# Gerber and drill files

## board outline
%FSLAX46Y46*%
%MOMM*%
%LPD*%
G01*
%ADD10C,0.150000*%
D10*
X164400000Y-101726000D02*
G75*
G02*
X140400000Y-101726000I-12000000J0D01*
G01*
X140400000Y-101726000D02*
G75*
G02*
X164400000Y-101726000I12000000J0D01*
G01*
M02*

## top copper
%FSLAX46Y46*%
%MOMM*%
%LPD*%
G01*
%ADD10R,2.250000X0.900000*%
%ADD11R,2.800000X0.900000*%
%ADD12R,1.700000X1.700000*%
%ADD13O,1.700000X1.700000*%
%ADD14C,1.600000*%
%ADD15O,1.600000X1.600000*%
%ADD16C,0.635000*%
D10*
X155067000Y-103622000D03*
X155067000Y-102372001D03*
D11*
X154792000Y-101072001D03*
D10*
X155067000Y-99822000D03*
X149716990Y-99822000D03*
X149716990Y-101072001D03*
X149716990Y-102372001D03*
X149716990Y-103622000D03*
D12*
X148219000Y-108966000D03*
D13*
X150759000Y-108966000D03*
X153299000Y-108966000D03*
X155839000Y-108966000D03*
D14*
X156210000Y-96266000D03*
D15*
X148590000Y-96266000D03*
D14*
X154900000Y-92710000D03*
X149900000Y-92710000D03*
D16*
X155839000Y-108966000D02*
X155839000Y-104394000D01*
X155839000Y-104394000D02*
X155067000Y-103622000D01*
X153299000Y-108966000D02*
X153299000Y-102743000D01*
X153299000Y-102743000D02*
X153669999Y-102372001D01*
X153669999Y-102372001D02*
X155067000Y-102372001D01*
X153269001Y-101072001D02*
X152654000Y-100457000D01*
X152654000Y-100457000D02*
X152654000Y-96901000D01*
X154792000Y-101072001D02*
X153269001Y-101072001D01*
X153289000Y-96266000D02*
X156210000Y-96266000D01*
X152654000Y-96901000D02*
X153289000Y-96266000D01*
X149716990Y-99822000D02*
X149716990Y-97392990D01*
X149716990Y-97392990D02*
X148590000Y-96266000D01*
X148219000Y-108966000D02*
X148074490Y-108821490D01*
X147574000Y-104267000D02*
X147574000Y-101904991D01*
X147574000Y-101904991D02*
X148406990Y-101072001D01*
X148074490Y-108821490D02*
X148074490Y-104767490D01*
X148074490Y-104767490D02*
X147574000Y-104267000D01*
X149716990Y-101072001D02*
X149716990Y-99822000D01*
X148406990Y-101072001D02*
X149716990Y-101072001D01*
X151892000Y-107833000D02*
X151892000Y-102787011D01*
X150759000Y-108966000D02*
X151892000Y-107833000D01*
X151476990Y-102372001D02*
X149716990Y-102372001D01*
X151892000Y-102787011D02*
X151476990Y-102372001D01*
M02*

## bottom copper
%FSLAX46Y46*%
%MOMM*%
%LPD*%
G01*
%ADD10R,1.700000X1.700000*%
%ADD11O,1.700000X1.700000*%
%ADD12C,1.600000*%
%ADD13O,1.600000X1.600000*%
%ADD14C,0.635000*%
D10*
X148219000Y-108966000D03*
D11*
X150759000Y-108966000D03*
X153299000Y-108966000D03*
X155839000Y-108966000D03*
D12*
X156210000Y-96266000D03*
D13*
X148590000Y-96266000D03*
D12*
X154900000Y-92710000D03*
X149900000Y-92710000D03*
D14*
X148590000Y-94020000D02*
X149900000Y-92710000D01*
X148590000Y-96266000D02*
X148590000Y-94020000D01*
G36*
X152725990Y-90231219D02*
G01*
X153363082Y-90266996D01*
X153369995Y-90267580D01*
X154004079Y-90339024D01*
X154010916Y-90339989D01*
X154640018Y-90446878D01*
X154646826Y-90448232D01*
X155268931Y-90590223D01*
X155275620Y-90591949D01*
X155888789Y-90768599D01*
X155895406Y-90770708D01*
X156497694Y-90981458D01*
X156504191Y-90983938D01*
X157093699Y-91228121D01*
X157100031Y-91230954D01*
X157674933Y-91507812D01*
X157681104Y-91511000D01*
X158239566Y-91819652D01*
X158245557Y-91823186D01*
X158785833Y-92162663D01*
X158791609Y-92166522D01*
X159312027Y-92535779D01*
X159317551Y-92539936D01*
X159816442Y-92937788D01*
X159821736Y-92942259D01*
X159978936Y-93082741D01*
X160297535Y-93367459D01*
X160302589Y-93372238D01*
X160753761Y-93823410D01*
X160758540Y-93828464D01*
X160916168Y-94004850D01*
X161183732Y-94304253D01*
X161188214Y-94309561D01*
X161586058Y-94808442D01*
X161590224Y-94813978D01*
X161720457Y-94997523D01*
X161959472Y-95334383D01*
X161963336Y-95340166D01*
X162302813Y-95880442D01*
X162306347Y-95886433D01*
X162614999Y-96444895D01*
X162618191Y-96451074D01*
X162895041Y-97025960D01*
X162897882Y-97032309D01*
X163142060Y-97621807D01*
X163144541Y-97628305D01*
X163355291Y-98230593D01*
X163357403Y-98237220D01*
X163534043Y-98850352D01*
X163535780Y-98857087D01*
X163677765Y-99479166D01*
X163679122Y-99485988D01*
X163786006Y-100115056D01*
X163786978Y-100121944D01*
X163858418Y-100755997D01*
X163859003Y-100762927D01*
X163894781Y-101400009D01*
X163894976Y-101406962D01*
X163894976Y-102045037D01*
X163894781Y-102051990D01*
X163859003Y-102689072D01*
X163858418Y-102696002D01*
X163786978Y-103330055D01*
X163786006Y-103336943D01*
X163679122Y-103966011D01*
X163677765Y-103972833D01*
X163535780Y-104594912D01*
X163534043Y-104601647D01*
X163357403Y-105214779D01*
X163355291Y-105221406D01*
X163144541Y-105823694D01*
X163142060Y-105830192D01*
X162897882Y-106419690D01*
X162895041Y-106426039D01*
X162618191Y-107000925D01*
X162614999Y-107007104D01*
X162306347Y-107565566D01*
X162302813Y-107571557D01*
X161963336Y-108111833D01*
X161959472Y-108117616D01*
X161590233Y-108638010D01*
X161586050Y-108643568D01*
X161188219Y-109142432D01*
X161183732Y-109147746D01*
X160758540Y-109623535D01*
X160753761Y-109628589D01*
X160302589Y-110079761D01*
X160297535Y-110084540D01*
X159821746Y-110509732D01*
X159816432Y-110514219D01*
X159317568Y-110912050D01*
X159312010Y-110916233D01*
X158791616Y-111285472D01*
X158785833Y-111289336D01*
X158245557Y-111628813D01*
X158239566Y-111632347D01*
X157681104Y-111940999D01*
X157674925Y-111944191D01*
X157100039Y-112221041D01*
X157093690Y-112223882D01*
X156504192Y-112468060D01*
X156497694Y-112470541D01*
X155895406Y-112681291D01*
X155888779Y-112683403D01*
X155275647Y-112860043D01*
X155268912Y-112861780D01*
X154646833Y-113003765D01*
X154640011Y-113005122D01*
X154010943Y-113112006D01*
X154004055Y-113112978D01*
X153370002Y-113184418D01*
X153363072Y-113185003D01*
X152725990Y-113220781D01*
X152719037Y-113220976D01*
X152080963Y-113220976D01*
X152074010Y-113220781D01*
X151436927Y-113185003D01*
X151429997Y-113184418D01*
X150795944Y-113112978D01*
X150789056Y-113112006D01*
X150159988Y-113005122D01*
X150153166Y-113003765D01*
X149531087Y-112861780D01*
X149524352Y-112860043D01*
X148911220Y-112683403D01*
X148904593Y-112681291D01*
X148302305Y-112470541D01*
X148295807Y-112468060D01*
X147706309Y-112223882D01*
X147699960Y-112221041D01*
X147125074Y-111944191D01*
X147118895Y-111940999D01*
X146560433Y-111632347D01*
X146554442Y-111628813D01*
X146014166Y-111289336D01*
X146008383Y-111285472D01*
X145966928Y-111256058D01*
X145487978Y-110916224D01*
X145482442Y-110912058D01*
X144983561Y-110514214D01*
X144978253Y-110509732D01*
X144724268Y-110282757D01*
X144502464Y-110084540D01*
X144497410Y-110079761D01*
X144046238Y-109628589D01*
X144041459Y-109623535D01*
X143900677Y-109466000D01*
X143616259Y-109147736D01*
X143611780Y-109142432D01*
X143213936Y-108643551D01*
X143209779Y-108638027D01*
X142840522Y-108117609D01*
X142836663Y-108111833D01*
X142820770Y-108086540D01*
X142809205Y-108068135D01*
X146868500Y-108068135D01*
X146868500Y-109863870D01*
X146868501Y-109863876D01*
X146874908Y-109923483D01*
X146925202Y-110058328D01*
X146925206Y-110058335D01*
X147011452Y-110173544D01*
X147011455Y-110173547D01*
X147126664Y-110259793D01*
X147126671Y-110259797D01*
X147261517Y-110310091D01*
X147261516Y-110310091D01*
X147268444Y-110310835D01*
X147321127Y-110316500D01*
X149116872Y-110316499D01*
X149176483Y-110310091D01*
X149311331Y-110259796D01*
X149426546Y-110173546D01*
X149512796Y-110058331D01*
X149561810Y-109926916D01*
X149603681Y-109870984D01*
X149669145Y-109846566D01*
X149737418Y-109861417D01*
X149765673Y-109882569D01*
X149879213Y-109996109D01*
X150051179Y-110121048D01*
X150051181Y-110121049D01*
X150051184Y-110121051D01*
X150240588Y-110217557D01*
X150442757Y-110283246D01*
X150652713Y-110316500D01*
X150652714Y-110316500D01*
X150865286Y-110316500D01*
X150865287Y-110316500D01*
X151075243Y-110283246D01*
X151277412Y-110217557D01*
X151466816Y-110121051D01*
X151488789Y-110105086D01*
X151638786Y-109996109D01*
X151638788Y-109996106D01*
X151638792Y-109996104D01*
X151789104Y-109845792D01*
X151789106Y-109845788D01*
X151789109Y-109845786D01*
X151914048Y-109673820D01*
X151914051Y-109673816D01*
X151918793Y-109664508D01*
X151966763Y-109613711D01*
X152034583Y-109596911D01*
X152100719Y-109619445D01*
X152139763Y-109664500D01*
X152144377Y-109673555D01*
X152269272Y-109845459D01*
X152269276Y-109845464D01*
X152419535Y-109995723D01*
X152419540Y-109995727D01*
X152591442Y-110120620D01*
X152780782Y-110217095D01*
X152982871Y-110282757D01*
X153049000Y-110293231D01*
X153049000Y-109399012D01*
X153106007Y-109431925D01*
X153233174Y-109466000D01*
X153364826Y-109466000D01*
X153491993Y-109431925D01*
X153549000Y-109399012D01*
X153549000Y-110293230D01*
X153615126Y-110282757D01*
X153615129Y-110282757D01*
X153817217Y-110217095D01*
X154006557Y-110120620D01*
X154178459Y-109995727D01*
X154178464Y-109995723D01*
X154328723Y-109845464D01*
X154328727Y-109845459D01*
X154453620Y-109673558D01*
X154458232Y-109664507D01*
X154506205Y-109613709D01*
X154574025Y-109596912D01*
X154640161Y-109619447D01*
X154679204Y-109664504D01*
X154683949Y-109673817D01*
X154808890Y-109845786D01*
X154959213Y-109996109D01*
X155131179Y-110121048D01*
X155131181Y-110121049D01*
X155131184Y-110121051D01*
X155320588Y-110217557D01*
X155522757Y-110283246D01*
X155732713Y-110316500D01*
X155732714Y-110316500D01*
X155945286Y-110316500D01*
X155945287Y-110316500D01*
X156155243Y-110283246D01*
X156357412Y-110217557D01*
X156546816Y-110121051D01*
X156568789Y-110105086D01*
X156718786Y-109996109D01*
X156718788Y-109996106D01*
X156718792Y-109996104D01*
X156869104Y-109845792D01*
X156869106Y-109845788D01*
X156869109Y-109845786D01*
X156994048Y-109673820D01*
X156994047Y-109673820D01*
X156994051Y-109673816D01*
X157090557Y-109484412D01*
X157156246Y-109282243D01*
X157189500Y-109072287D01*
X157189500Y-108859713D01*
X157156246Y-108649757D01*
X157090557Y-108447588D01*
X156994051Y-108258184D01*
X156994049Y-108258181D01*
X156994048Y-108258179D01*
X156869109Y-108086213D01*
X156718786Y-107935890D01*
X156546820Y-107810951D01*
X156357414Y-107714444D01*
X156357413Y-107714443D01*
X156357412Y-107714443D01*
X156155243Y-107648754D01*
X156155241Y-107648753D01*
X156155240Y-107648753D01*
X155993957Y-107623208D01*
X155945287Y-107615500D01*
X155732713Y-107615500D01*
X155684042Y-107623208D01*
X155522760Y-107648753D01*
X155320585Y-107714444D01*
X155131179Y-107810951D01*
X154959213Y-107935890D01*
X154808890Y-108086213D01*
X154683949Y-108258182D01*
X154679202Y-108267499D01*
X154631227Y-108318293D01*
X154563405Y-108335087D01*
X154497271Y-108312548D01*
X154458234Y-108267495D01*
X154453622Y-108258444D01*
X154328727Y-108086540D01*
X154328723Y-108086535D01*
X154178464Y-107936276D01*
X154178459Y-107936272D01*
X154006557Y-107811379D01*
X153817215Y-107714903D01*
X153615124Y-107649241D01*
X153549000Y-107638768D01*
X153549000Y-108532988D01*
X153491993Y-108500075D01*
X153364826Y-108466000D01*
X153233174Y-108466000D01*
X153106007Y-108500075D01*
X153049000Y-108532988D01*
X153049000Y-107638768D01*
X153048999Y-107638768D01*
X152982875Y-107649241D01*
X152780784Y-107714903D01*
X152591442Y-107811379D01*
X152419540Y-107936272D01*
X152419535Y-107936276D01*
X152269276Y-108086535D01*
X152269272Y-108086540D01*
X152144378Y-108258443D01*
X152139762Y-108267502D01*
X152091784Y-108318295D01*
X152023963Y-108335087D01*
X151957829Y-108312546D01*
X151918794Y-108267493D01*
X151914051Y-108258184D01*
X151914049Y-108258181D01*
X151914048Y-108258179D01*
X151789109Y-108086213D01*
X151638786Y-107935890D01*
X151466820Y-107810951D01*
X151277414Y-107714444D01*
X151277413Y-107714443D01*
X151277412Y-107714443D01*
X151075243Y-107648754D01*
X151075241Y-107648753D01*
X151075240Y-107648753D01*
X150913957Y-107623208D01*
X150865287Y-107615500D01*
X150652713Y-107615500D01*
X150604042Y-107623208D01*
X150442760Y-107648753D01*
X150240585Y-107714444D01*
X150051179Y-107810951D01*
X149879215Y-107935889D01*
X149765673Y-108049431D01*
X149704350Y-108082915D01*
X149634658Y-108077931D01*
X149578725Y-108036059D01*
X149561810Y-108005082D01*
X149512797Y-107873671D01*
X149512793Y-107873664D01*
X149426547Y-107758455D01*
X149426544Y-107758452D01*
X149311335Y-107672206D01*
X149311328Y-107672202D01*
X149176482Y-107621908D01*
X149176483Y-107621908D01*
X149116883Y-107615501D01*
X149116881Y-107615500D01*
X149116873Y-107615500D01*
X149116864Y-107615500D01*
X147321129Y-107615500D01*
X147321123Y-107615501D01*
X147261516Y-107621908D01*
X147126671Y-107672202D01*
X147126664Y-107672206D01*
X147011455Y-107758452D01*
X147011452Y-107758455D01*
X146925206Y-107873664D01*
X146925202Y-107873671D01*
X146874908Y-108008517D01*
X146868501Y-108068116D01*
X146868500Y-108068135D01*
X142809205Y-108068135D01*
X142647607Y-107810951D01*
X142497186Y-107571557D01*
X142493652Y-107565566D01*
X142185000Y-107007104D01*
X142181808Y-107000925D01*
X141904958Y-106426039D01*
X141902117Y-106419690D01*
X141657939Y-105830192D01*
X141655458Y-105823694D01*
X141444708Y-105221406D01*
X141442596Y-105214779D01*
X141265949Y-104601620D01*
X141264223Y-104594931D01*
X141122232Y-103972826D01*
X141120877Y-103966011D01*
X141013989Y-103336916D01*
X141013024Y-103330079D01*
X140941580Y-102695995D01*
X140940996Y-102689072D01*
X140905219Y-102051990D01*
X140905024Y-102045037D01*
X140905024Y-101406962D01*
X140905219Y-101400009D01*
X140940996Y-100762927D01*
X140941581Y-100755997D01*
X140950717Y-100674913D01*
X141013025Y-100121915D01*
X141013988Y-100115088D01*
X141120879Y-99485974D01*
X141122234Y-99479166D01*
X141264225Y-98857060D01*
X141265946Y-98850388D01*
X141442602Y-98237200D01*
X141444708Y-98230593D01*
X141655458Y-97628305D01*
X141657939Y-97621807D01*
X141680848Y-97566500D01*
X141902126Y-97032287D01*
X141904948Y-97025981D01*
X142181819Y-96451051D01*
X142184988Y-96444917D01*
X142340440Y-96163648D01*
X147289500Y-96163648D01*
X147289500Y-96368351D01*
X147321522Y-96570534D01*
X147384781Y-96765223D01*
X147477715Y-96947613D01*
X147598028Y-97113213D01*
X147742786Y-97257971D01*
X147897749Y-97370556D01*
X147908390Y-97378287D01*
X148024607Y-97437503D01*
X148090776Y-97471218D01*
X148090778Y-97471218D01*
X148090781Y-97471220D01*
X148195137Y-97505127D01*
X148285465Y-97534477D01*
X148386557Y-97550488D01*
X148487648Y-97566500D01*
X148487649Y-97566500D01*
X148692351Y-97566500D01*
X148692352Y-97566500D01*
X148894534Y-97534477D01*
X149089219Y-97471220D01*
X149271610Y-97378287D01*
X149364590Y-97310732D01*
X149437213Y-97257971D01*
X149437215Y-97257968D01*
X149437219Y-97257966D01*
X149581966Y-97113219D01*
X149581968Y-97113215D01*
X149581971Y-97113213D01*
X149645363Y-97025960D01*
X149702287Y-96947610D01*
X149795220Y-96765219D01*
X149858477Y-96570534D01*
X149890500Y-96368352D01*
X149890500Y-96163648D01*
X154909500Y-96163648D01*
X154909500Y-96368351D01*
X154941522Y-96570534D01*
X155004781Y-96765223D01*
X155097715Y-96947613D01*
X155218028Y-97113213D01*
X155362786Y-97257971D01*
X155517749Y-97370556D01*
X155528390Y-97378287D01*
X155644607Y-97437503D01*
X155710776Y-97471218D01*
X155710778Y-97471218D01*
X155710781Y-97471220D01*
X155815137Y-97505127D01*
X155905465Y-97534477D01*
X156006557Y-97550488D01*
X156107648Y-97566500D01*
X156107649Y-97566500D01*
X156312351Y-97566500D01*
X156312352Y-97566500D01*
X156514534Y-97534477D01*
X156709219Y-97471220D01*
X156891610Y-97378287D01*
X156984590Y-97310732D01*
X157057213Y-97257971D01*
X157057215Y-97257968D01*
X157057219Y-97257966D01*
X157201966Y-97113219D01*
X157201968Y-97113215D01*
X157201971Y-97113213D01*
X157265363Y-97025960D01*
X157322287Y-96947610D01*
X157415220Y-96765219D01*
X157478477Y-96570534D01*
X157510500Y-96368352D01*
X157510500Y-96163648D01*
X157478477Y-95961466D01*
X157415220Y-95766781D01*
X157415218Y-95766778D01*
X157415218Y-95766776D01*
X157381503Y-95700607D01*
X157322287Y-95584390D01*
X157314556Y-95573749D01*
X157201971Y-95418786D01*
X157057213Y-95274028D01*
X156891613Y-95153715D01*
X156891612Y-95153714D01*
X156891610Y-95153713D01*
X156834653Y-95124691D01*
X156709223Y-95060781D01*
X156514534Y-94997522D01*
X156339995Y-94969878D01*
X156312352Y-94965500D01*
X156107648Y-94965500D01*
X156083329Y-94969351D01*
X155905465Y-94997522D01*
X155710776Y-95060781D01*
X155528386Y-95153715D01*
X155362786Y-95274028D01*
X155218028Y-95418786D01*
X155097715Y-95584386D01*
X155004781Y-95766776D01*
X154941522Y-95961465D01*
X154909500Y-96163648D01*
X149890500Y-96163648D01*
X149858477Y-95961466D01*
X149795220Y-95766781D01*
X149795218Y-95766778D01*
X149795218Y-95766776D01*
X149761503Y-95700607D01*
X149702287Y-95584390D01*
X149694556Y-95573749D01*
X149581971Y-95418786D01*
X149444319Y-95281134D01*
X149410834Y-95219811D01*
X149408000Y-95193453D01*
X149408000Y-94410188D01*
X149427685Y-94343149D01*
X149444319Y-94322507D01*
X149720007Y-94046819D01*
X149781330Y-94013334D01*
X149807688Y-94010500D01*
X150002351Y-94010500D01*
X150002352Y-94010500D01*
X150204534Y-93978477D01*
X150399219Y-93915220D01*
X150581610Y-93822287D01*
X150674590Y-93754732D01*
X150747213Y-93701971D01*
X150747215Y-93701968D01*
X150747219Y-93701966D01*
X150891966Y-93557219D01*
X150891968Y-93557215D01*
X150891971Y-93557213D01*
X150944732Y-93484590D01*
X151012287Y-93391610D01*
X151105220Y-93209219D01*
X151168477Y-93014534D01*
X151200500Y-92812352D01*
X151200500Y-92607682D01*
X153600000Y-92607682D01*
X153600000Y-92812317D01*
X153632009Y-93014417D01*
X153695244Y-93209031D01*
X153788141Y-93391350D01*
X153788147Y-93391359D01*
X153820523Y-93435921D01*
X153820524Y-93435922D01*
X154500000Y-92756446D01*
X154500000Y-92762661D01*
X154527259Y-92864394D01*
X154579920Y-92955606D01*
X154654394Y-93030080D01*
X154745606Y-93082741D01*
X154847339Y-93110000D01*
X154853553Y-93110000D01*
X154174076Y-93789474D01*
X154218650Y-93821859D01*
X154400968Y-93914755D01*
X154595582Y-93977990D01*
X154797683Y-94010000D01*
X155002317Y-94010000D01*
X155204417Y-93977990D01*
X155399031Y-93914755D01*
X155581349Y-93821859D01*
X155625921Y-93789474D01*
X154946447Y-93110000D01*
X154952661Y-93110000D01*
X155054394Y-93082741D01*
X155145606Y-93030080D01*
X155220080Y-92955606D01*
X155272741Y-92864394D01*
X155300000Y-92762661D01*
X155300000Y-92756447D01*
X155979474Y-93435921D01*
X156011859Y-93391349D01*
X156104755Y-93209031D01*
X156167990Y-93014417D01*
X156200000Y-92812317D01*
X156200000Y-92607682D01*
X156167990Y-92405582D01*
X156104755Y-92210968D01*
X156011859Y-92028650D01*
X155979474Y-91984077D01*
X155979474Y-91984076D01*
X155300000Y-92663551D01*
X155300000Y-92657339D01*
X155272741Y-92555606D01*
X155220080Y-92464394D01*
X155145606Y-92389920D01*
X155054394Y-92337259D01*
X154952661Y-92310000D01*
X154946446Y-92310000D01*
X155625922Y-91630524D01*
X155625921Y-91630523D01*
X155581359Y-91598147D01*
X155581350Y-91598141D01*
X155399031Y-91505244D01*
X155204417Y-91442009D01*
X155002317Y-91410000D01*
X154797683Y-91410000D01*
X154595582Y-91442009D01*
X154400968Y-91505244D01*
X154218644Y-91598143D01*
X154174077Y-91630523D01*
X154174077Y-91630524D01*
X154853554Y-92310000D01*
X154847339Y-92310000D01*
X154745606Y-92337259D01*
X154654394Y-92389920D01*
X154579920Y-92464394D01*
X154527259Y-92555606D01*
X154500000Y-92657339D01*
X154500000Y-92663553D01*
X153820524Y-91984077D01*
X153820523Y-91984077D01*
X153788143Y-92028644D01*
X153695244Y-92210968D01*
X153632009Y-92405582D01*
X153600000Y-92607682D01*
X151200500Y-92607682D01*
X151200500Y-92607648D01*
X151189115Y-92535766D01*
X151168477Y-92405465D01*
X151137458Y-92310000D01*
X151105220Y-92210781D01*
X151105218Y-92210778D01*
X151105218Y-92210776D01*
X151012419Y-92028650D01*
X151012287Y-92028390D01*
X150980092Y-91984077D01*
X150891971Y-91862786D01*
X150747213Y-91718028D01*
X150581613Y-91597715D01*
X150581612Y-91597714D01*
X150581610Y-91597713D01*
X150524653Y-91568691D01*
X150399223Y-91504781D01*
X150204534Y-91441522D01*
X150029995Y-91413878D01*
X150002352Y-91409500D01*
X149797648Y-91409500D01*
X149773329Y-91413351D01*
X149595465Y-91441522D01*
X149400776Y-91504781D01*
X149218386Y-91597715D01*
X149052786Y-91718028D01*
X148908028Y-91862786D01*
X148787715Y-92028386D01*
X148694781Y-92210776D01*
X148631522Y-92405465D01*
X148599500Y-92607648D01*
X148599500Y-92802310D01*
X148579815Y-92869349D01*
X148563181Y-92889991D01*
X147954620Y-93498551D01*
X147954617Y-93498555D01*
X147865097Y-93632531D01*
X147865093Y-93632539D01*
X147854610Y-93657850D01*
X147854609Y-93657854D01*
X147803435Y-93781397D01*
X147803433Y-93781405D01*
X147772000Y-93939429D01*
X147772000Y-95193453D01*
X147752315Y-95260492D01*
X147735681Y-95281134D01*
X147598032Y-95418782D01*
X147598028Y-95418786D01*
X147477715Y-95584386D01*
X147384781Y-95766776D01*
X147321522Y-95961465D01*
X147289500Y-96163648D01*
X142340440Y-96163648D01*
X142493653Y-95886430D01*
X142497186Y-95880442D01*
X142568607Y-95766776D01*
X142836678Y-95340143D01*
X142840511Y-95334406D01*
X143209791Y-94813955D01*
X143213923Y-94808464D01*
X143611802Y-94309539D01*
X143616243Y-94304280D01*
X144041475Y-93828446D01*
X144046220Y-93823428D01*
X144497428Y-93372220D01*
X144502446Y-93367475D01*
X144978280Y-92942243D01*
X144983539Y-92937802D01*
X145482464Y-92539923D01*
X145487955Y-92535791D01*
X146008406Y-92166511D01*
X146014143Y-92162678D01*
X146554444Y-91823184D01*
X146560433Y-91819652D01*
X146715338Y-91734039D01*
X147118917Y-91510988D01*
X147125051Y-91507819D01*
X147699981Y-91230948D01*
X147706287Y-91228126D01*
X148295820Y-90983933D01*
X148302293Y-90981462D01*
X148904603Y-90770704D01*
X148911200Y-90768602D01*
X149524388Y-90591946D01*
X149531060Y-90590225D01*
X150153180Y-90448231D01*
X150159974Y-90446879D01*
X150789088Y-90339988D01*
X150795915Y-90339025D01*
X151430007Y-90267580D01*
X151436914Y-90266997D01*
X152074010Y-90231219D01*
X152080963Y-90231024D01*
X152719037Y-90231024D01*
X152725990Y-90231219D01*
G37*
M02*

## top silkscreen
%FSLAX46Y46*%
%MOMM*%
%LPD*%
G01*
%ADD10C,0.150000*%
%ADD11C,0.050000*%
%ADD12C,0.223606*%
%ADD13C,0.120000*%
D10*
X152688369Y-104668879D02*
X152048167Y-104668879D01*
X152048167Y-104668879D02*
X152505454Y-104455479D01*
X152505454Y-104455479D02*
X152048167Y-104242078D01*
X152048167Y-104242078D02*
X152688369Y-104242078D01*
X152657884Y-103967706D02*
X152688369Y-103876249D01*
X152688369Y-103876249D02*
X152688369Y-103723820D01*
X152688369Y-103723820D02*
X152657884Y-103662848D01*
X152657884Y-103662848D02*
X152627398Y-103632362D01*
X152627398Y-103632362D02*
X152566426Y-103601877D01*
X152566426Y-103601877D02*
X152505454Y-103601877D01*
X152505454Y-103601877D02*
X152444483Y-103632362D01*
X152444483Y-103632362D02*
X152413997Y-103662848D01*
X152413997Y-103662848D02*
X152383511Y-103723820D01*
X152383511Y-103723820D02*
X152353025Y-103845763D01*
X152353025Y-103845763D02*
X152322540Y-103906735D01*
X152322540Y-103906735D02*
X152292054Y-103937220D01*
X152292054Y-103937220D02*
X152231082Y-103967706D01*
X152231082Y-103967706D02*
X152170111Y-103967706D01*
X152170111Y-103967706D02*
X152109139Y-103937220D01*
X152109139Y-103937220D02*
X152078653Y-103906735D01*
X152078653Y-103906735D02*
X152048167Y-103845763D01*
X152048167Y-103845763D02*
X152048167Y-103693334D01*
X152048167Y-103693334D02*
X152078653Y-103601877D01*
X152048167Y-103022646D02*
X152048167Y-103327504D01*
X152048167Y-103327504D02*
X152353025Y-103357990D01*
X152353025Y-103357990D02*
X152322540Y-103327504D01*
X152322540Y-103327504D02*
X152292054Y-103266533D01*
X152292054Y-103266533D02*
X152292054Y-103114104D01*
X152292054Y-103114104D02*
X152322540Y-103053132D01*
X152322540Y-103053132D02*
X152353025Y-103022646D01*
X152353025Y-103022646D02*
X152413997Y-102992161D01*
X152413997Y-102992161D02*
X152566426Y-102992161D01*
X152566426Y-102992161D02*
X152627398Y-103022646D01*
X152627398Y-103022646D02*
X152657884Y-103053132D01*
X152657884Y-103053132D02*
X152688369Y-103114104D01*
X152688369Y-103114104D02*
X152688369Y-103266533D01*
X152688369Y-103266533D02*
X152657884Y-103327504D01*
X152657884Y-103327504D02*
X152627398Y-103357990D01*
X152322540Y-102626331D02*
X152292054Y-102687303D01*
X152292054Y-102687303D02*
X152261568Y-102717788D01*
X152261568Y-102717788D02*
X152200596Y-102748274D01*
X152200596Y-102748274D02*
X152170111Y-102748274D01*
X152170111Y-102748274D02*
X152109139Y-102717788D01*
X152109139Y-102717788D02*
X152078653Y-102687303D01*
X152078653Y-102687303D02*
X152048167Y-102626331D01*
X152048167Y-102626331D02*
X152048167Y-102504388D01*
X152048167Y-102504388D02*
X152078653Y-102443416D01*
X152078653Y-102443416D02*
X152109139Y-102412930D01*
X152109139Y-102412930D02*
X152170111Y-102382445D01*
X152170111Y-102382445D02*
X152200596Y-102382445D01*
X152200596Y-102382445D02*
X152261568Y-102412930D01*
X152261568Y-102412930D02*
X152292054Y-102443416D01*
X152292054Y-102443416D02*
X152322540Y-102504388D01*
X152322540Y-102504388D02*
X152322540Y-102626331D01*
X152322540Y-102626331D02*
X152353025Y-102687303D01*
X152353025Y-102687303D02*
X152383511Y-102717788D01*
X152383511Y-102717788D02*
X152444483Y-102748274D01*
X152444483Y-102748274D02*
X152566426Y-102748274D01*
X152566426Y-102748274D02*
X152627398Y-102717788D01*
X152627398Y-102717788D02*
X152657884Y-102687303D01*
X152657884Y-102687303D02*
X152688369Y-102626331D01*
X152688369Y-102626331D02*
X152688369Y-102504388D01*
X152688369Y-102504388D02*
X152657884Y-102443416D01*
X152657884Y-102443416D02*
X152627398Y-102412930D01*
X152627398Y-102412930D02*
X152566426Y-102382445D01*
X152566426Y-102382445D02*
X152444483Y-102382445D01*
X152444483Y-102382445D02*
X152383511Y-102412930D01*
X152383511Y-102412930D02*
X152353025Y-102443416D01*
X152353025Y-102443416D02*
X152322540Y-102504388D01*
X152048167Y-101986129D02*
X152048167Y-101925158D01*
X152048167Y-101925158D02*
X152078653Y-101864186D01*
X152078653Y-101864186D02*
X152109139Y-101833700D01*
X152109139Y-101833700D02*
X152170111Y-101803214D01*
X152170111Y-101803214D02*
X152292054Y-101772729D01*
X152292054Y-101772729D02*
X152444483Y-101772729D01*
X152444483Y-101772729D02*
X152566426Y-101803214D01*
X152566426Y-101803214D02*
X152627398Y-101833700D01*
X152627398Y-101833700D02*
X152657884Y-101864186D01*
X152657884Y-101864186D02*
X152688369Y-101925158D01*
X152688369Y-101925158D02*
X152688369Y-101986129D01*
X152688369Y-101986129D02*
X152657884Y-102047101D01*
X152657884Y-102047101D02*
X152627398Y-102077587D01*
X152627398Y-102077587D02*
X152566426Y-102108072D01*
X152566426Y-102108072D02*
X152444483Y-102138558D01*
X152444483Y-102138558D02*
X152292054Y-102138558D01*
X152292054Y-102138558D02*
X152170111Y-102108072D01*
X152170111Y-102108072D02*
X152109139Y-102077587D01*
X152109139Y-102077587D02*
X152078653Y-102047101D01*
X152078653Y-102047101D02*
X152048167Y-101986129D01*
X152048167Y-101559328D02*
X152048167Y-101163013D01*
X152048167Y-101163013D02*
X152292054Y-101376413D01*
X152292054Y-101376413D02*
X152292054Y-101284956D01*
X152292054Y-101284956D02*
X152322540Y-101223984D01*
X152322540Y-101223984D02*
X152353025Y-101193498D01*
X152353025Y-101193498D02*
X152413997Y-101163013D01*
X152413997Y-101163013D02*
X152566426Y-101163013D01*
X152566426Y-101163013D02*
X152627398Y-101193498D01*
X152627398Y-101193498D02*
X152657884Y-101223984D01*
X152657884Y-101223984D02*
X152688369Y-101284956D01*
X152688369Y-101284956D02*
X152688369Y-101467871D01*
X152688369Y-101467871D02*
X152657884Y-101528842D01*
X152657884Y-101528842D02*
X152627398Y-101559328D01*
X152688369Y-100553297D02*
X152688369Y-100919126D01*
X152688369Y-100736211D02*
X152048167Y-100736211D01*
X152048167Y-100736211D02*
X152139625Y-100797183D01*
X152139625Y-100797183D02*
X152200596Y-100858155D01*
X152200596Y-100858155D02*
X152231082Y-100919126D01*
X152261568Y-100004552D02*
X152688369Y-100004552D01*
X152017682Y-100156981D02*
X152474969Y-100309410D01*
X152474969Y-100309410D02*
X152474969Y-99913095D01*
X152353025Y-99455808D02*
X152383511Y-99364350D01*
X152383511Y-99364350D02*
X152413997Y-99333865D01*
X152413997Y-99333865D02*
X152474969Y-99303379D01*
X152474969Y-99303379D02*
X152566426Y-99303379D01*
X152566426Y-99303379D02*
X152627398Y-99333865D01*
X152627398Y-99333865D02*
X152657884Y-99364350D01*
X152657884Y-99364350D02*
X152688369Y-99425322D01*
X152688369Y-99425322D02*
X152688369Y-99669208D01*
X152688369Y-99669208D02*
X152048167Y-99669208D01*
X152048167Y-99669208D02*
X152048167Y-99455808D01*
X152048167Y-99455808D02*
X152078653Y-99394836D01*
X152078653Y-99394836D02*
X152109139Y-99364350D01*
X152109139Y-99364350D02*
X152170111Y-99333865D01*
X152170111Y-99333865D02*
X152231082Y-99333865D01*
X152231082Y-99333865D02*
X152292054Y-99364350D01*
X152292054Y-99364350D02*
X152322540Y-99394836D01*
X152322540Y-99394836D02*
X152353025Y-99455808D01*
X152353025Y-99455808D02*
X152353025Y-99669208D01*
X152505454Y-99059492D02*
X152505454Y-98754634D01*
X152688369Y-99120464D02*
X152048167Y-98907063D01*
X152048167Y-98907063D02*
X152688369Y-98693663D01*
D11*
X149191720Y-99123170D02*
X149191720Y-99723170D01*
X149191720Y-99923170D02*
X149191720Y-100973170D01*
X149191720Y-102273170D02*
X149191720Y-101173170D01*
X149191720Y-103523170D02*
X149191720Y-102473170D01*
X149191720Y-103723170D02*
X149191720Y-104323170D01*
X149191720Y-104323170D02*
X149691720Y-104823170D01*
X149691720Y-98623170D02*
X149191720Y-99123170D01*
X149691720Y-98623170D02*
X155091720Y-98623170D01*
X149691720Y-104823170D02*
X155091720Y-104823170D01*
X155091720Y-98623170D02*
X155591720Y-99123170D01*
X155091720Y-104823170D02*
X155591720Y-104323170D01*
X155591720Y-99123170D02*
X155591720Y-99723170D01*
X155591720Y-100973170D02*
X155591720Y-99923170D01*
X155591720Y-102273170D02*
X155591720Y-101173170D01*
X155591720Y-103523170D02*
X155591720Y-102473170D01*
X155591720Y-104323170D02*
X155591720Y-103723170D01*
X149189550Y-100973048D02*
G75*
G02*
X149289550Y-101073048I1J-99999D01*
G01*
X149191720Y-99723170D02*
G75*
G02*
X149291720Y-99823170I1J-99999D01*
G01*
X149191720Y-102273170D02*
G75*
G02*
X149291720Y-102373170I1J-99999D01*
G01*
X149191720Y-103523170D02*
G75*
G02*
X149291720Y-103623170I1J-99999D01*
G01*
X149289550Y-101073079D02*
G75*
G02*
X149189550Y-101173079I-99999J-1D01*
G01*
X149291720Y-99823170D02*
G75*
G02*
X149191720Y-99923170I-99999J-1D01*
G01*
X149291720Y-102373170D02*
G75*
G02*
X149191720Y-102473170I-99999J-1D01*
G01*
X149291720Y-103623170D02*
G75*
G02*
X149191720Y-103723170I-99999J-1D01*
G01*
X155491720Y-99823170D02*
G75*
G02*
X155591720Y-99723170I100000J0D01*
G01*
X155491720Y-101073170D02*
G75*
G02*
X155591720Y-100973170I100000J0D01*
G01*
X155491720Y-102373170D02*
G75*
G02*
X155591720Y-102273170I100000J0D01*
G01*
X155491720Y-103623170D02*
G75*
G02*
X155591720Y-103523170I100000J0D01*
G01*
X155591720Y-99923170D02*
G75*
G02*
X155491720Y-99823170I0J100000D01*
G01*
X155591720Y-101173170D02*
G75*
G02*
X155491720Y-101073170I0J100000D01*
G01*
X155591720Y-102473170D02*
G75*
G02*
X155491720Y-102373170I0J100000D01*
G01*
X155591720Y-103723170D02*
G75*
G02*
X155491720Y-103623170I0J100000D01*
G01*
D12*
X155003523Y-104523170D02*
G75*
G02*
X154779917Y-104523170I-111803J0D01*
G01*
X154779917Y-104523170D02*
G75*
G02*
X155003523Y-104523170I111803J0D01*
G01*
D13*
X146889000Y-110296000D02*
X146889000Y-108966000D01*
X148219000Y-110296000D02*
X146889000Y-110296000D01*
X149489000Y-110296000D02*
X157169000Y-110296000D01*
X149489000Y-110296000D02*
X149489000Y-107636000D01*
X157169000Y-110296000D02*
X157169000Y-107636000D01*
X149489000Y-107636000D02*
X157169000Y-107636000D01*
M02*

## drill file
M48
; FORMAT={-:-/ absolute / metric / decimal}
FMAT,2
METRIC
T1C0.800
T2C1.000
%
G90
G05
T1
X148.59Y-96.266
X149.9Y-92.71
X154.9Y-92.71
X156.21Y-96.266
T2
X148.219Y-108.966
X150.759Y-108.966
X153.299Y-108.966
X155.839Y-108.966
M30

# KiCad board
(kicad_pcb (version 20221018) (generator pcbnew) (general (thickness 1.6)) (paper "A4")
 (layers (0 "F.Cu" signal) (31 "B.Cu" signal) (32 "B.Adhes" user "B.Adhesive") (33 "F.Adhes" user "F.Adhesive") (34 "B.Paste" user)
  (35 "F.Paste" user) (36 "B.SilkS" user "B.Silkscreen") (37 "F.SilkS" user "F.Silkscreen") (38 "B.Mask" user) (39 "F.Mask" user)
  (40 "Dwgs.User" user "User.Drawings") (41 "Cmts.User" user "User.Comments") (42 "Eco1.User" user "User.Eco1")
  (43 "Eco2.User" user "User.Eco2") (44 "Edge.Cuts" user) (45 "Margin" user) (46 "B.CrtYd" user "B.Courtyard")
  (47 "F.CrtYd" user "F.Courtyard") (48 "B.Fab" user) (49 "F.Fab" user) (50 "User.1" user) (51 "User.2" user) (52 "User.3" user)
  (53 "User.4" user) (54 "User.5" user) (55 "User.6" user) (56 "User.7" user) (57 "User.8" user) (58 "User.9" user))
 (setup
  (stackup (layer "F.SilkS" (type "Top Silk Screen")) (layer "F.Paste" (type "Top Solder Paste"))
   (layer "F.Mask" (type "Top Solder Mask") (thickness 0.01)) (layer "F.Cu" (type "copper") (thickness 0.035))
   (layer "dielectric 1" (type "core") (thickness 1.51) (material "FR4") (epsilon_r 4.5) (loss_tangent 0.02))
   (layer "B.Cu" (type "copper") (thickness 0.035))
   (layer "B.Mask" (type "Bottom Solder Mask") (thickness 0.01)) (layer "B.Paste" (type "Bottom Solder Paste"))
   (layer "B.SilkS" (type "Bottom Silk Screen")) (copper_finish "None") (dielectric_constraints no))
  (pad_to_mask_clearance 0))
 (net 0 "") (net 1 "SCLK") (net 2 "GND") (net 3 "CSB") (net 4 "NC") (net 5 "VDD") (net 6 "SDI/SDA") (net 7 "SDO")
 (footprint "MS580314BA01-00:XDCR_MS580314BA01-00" (layer "F.Cu") (at 152.39172 101.72317)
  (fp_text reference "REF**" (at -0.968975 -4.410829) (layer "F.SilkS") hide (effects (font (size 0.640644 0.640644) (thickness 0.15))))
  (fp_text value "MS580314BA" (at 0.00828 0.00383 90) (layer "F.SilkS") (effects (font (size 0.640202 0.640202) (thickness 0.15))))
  (fp_line (start -3.2 -2.6) (end -3.2 -2) (stroke (width 0.05) (type solid)) (layer "F.SilkS"))
  (fp_line (start -3.2 -1.8) (end -3.2 -0.75) (stroke (width 0.05) (type solid)) (layer "F.SilkS"))
  (fp_line (start -3.2 0.55) (end -3.2 -0.55) (stroke (width 0.05) (type solid)) (layer "F.SilkS"))
  (fp_line (start -3.2 1.8) (end -3.2 0.75) (stroke (width 0.05) (type solid)) (layer "F.SilkS"))
  (fp_line (start -3.2 2) (end -3.2 2.6) (stroke (width 0.05) (type solid)) (layer "F.SilkS"))
  (fp_line (start -3.2 2.6) (end -2.7 3.1) (stroke (width 0.05) (type solid)) (layer "F.SilkS"))
  (fp_line (start -2.7 -3.1) (end -3.2 -2.6) (stroke (width 0.05) (type solid)) (layer "F.SilkS"))
  (fp_line (start -2.7 -3.1) (end 2.7 -3.1) (stroke (width 0.05) (type solid)) (layer "F.SilkS"))
  (fp_line (start -2.7 3.1) (end 2.7 3.1) (stroke (width 0.05) (type solid)) (layer "F.SilkS"))
  (fp_line (start 2.7 -3.1) (end 3.2 -2.6) (stroke (width 0.05) (type solid)) (layer "F.SilkS"))
  (fp_line (start 2.7 3.1) (end 3.2 2.6) (stroke (width 0.05) (type solid)) (layer "F.SilkS"))
  (fp_line (start 3.2 -2.6) (end 3.2 -2) (stroke (width 0.05) (type solid)) (layer "F.SilkS"))
  (fp_line (start 3.2 -0.75) (end 3.2 -1.8) (stroke (width 0.05) (type solid)) (layer "F.SilkS"))
  (fp_line (start 3.2 0.55) (end 3.2 -0.55) (stroke (width 0.05) (type solid)) (layer "F.SilkS"))
  (fp_line (start 3.2 1.8) (end 3.2 0.75) (stroke (width 0.05) (type solid)) (layer "F.SilkS"))
  (fp_line (start 3.2 2.6) (end 3.2 2) (stroke (width 0.05) (type solid)) (layer "F.SilkS"))
  (fp_arc (start -3.20217 -0.750122) (mid -3.131459 -0.720833) (end -3.10217 -0.650122) (stroke (width 0.05) (type solid)) (layer "F.SilkS"))
  (fp_arc (start -3.2 -2) (mid -3.129289 -1.970711) (end -3.1 -1.9) (stroke (width 0.05) (type solid)) (layer "F.SilkS"))
  (fp_arc (start -3.2 0.55) (mid -3.129289 0.579289) (end -3.1 0.65) (stroke (width 0.05) (type solid)) (layer "F.SilkS"))
  (fp_arc (start -3.2 1.8) (mid -3.129289 1.829289) (end -3.1 1.9) (stroke (width 0.05) (type solid)) (layer "F.SilkS"))
  (fp_arc (start -3.10217 -0.650091) (mid -3.131459 -0.57938) (end -3.20217 -0.550091) (stroke (width 0.05) (type solid)) (layer "F.SilkS"))
  (fp_arc (start -3.1 -1.9) (mid -3.129289 -1.829289) (end -3.2 -1.8) (stroke (width 0.05) (type solid)) (layer "F.SilkS"))
  (fp_arc (start -3.1 0.65) (mid -3.129289 0.720711) (end -3.2 0.75) (stroke (width 0.05) (type solid)) (layer "F.SilkS"))
  (fp_arc (start -3.1 1.9) (mid -3.129289 1.970711) (end -3.2 2) (stroke (width 0.05) (type solid)) (layer "F.SilkS"))
  (fp_arc (start 3.1 -1.9) (mid 3.129289 -1.970711) (end 3.2 -2) (stroke (width 0.05) (type solid)) (layer "F.SilkS"))
  (fp_arc (start 3.1 -0.65) (mid 3.129289 -0.720711) (end 3.2 -0.75) (stroke (width 0.05) (type solid)) (layer "F.SilkS"))
  (fp_arc (start 3.1 0.65) (mid 3.129289 0.579289) (end 3.2 0.55) (stroke (width 0.05) (type solid)) (layer "F.SilkS"))
  (fp_arc (start 3.1 1.9) (mid 3.129289 1.829289) (end 3.2 1.8) (stroke (width 0.05) (type solid)) (layer "F.SilkS"))
  (fp_arc (start 3.2 -1.8) (mid 3.129289 -1.829289) (end 3.1 -1.9) (stroke (width 0.05) (type solid)) (layer "F.SilkS"))
  (fp_arc (start 3.2 -0.55) (mid 3.129289 -0.579289) (end 3.1 -0.65) (stroke (width 0.05) (type solid)) (layer "F.SilkS"))
  (fp_arc (start 3.2 0.75) (mid 3.129289 0.720711) (end 3.1 0.65) (stroke (width 0.05) (type solid)) (layer "F.SilkS"))
  (fp_arc (start 3.2 2) (mid 3.129289 1.970711) (end 3.1 1.9) (stroke (width 0.05) (type solid)) (layer "F.SilkS"))
  (fp_circle (center 2.5 2.8) (end 2.723606 2.8) (stroke (width 0) (type solid)) (fill solid) (layer "F.SilkS"))
  (pad "1" smd rect (at 2.67528 1.89883) (size 2.25 0.9) (layers "F.Cu" "F.Paste" "F.Mask") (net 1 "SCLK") (solder_mask_margin 0.102))
  (pad "2" smd rect (at 2.67528 0.648831) (size 2.25 0.9) (layers "F.Cu" "F.Paste" "F.Mask") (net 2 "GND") (solder_mask_margin 0.102))
  (pad "3" smd rect (at 2.40028 -0.651169) (size 2.8 0.9) (layers "F.Cu" "F.Paste" "F.Mask") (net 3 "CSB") (solder_mask_margin 0.102))
  (pad "4" smd rect (at 2.67528 -1.90117) (size 2.25 0.9) (layers "F.Cu" "F.Paste" "F.Mask") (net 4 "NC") (solder_mask_margin 0.102))
  (pad "5" smd rect (at -2.67473 -1.90117) (size 2.25 0.9) (layers "F.Cu" "F.Paste" "F.Mask") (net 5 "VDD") (solder_mask_margin 0.102))
  (pad "6" smd rect (at -2.67473 -0.651169) (size 2.25 0.9) (layers "F.Cu" "F.Paste" "F.Mask") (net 5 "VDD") (solder_mask_margin 0.102))
  (pad "7" smd rect (at -2.67473 0.648831) (size 2.25 0.9) (layers "F.Cu" "F.Paste" "F.Mask") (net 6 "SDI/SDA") (solder_mask_margin 0.102))
  (pad "8" smd rect (at -2.67473 1.89883) (size 2.25 0.9) (layers "F.Cu" "F.Paste" "F.Mask") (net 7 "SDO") (solder_mask_margin 0.102)))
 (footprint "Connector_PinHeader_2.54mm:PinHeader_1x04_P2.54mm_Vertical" (layer "F.Cu") (at 148.219 108.966 90)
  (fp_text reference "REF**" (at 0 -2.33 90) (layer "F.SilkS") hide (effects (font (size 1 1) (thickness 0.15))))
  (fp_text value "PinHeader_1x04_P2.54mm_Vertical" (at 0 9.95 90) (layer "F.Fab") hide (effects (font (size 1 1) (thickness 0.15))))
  (fp_line (start -1.33 -1.33) (end 0 -1.33) (stroke (width 0.12) (type solid)) (layer "F.SilkS"))
  (fp_line (start -1.33 0) (end -1.33 -1.33) (stroke (width 0.12) (type solid)) (layer "F.SilkS"))
  (fp_line (start -1.33 1.27) (end -1.33 8.95) (stroke (width 0.12) (type solid)) (layer "F.SilkS"))
  (fp_line (start -1.33 1.27) (end 1.33 1.27) (stroke (width 0.12) (type solid)) (layer "F.SilkS"))
  (fp_line (start -1.33 8.95) (end 1.33 8.95) (stroke (width 0.12) (type solid)) (layer "F.SilkS"))
  (fp_line (start 1.33 1.27) (end 1.33 8.95) (stroke (width 0.12) (type solid)) (layer "F.SilkS"))
  (pad "1" thru_hole rect (at 0 0 90) (size 1.7 1.7) (drill 1) (layers "*.Cu" "*.Mask") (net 5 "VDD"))
  (pad "2" thru_hole oval (at 0 2.54 90) (size 1.7 1.7) (drill 1) (layers "*.Cu" "*.Mask") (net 6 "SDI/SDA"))
  (pad "3" thru_hole oval (at 0 5.08 90) (size 1.7 1.7) (drill 1) (layers "*.Cu" "*.Mask") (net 2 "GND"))
  (pad "4" thru_hole oval (at 0 7.62 90) (size 1.7 1.7) (drill 1) (layers "*.Cu" "*.Mask") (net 1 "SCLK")))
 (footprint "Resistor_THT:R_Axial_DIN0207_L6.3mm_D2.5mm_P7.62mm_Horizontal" (layer "B.Cu") (at 156.21 96.266 180)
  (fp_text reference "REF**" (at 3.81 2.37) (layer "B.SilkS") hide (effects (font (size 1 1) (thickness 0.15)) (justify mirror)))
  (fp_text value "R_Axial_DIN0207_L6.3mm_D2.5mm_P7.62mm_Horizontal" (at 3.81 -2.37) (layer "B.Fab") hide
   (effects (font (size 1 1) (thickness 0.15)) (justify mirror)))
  (pad "1" thru_hole circle (at 0 0 180) (size 1.6 1.6) (drill 0.8) (layers "*.Cu" "*.Mask") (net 3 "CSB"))
  (pad "2" thru_hole oval (at 7.62 0 180) (size 1.6 1.6) (drill 0.8) (layers "*.Cu" "*.Mask") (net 5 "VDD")))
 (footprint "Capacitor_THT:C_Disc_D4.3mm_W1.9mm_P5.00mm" (layer "B.Cu") (at 154.9 92.71 180)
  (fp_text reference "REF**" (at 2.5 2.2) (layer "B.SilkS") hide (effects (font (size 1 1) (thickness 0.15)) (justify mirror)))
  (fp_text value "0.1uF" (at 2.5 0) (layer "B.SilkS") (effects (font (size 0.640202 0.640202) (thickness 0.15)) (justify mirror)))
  (pad "1" thru_hole circle (at 0 0 180) (size 1.6 1.6) (drill 0.8) (layers "*.Cu" "*.Mask") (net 2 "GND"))
  (pad "2" thru_hole circle (at 5 0 180) (size 1.6 1.6) (drill 0.8) (layers "*.Cu" "*.Mask") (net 5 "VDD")))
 (gr_circle (center 152.4 101.726) (end 164.4 101.726) (stroke (width 0.15) (type default)) (fill none) (layer "Edge.Cuts"))
 (segment (start 155.839 108.966) (end 155.839 104.394) (width 0.635) (layer "F.Cu") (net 1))
 (segment (start 155.839 104.394) (end 155.067 103.622) (width 0.635) (layer "F.Cu") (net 1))
 (segment (start 153.299 108.966) (end 153.299 102.743) (width 0.635) (layer "F.Cu") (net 2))
 (segment (start 153.299 102.743) (end 153.669999 102.372001) (width 0.635) (layer "F.Cu") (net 2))
 (segment (start 153.669999 102.372001) (end 155.067 102.372001) (width 0.635) (layer "F.Cu") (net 2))
 (segment (start 153.269001 101.072001) (end 152.654 100.457) (width 0.635) (layer "F.Cu") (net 3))
 (segment (start 152.654 100.457) (end 152.654 96.901) (width 0.635) (layer "F.Cu") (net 3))
 (segment (start 154.792 101.072001) (end 153.269001 101.072001) (width 0.635) (layer "F.Cu") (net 3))
 (segment (start 153.289 96.266) (end 156.21 96.266) (width 0.635) (layer "F.Cu") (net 3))
 (segment (start 152.654 96.901) (end 153.289 96.266) (width 0.635) (layer "F.Cu") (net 3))
 (segment (start 149.71699 99.822) (end 149.71699 97.39299) (width 0.635) (layer "F.Cu") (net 5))
 (segment (start 149.71699 97.39299) (end 148.59 96.266) (width 0.635) (layer "F.Cu") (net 5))
 (segment (start 148.219 108.966) (end 148.07449 108.82149) (width 0.635) (layer "F.Cu") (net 5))
 (segment (start 147.574 104.267) (end 147.574 101.904991) (width 0.635) (layer "F.Cu") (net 5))
 (segment (start 147.574 101.904991) (end 148.40699 101.072001) (width 0.635) (layer "F.Cu") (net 5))
 (segment (start 148.07449 108.82149) (end 148.07449 104.76749) (width 0.635) (layer "F.Cu") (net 5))
 (segment (start 148.07449 104.76749) (end 147.574 104.267) (width 0.635) (layer "F.Cu") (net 5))
 (segment (start 149.71699 101.072001) (end 149.71699 99.822) (width 0.635) (layer "F.Cu") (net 5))
 (segment (start 148.40699 101.072001) (end 149.71699 101.072001) (width 0.635) (layer "F.Cu") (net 5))
 (segment (start 148.59 94.02) (end 149.9 92.71) (width 0.635) (layer "B.Cu") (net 5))
 (segment (start 148.59 96.266) (end 148.59 94.02) (width 0.635) (layer "B.Cu") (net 5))
 (segment (start 151.892 107.833) (end 151.892 102.787011) (width 0.635) (layer "F.Cu") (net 6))
 (segment (start 150.759 108.966) (end 151.892 107.833) (width 0.635) (layer "F.Cu") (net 6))
 (segment (start 151.47699 102.372001) (end 149.71699 102.372001) (width 0.635) (layer "F.Cu") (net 6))
 (segment (start 151.892 102.787011) (end 151.47699 102.372001) (width 0.635) (layer "F.Cu") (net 6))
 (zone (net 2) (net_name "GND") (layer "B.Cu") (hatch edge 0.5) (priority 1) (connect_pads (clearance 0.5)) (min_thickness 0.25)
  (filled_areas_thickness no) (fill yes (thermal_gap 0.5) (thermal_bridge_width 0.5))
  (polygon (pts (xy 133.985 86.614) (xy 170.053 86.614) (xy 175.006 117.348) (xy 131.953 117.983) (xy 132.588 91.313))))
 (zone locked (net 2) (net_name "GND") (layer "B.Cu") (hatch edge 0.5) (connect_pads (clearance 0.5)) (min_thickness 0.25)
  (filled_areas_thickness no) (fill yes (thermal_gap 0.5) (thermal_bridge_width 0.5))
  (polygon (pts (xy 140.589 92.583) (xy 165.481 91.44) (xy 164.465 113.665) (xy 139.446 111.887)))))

